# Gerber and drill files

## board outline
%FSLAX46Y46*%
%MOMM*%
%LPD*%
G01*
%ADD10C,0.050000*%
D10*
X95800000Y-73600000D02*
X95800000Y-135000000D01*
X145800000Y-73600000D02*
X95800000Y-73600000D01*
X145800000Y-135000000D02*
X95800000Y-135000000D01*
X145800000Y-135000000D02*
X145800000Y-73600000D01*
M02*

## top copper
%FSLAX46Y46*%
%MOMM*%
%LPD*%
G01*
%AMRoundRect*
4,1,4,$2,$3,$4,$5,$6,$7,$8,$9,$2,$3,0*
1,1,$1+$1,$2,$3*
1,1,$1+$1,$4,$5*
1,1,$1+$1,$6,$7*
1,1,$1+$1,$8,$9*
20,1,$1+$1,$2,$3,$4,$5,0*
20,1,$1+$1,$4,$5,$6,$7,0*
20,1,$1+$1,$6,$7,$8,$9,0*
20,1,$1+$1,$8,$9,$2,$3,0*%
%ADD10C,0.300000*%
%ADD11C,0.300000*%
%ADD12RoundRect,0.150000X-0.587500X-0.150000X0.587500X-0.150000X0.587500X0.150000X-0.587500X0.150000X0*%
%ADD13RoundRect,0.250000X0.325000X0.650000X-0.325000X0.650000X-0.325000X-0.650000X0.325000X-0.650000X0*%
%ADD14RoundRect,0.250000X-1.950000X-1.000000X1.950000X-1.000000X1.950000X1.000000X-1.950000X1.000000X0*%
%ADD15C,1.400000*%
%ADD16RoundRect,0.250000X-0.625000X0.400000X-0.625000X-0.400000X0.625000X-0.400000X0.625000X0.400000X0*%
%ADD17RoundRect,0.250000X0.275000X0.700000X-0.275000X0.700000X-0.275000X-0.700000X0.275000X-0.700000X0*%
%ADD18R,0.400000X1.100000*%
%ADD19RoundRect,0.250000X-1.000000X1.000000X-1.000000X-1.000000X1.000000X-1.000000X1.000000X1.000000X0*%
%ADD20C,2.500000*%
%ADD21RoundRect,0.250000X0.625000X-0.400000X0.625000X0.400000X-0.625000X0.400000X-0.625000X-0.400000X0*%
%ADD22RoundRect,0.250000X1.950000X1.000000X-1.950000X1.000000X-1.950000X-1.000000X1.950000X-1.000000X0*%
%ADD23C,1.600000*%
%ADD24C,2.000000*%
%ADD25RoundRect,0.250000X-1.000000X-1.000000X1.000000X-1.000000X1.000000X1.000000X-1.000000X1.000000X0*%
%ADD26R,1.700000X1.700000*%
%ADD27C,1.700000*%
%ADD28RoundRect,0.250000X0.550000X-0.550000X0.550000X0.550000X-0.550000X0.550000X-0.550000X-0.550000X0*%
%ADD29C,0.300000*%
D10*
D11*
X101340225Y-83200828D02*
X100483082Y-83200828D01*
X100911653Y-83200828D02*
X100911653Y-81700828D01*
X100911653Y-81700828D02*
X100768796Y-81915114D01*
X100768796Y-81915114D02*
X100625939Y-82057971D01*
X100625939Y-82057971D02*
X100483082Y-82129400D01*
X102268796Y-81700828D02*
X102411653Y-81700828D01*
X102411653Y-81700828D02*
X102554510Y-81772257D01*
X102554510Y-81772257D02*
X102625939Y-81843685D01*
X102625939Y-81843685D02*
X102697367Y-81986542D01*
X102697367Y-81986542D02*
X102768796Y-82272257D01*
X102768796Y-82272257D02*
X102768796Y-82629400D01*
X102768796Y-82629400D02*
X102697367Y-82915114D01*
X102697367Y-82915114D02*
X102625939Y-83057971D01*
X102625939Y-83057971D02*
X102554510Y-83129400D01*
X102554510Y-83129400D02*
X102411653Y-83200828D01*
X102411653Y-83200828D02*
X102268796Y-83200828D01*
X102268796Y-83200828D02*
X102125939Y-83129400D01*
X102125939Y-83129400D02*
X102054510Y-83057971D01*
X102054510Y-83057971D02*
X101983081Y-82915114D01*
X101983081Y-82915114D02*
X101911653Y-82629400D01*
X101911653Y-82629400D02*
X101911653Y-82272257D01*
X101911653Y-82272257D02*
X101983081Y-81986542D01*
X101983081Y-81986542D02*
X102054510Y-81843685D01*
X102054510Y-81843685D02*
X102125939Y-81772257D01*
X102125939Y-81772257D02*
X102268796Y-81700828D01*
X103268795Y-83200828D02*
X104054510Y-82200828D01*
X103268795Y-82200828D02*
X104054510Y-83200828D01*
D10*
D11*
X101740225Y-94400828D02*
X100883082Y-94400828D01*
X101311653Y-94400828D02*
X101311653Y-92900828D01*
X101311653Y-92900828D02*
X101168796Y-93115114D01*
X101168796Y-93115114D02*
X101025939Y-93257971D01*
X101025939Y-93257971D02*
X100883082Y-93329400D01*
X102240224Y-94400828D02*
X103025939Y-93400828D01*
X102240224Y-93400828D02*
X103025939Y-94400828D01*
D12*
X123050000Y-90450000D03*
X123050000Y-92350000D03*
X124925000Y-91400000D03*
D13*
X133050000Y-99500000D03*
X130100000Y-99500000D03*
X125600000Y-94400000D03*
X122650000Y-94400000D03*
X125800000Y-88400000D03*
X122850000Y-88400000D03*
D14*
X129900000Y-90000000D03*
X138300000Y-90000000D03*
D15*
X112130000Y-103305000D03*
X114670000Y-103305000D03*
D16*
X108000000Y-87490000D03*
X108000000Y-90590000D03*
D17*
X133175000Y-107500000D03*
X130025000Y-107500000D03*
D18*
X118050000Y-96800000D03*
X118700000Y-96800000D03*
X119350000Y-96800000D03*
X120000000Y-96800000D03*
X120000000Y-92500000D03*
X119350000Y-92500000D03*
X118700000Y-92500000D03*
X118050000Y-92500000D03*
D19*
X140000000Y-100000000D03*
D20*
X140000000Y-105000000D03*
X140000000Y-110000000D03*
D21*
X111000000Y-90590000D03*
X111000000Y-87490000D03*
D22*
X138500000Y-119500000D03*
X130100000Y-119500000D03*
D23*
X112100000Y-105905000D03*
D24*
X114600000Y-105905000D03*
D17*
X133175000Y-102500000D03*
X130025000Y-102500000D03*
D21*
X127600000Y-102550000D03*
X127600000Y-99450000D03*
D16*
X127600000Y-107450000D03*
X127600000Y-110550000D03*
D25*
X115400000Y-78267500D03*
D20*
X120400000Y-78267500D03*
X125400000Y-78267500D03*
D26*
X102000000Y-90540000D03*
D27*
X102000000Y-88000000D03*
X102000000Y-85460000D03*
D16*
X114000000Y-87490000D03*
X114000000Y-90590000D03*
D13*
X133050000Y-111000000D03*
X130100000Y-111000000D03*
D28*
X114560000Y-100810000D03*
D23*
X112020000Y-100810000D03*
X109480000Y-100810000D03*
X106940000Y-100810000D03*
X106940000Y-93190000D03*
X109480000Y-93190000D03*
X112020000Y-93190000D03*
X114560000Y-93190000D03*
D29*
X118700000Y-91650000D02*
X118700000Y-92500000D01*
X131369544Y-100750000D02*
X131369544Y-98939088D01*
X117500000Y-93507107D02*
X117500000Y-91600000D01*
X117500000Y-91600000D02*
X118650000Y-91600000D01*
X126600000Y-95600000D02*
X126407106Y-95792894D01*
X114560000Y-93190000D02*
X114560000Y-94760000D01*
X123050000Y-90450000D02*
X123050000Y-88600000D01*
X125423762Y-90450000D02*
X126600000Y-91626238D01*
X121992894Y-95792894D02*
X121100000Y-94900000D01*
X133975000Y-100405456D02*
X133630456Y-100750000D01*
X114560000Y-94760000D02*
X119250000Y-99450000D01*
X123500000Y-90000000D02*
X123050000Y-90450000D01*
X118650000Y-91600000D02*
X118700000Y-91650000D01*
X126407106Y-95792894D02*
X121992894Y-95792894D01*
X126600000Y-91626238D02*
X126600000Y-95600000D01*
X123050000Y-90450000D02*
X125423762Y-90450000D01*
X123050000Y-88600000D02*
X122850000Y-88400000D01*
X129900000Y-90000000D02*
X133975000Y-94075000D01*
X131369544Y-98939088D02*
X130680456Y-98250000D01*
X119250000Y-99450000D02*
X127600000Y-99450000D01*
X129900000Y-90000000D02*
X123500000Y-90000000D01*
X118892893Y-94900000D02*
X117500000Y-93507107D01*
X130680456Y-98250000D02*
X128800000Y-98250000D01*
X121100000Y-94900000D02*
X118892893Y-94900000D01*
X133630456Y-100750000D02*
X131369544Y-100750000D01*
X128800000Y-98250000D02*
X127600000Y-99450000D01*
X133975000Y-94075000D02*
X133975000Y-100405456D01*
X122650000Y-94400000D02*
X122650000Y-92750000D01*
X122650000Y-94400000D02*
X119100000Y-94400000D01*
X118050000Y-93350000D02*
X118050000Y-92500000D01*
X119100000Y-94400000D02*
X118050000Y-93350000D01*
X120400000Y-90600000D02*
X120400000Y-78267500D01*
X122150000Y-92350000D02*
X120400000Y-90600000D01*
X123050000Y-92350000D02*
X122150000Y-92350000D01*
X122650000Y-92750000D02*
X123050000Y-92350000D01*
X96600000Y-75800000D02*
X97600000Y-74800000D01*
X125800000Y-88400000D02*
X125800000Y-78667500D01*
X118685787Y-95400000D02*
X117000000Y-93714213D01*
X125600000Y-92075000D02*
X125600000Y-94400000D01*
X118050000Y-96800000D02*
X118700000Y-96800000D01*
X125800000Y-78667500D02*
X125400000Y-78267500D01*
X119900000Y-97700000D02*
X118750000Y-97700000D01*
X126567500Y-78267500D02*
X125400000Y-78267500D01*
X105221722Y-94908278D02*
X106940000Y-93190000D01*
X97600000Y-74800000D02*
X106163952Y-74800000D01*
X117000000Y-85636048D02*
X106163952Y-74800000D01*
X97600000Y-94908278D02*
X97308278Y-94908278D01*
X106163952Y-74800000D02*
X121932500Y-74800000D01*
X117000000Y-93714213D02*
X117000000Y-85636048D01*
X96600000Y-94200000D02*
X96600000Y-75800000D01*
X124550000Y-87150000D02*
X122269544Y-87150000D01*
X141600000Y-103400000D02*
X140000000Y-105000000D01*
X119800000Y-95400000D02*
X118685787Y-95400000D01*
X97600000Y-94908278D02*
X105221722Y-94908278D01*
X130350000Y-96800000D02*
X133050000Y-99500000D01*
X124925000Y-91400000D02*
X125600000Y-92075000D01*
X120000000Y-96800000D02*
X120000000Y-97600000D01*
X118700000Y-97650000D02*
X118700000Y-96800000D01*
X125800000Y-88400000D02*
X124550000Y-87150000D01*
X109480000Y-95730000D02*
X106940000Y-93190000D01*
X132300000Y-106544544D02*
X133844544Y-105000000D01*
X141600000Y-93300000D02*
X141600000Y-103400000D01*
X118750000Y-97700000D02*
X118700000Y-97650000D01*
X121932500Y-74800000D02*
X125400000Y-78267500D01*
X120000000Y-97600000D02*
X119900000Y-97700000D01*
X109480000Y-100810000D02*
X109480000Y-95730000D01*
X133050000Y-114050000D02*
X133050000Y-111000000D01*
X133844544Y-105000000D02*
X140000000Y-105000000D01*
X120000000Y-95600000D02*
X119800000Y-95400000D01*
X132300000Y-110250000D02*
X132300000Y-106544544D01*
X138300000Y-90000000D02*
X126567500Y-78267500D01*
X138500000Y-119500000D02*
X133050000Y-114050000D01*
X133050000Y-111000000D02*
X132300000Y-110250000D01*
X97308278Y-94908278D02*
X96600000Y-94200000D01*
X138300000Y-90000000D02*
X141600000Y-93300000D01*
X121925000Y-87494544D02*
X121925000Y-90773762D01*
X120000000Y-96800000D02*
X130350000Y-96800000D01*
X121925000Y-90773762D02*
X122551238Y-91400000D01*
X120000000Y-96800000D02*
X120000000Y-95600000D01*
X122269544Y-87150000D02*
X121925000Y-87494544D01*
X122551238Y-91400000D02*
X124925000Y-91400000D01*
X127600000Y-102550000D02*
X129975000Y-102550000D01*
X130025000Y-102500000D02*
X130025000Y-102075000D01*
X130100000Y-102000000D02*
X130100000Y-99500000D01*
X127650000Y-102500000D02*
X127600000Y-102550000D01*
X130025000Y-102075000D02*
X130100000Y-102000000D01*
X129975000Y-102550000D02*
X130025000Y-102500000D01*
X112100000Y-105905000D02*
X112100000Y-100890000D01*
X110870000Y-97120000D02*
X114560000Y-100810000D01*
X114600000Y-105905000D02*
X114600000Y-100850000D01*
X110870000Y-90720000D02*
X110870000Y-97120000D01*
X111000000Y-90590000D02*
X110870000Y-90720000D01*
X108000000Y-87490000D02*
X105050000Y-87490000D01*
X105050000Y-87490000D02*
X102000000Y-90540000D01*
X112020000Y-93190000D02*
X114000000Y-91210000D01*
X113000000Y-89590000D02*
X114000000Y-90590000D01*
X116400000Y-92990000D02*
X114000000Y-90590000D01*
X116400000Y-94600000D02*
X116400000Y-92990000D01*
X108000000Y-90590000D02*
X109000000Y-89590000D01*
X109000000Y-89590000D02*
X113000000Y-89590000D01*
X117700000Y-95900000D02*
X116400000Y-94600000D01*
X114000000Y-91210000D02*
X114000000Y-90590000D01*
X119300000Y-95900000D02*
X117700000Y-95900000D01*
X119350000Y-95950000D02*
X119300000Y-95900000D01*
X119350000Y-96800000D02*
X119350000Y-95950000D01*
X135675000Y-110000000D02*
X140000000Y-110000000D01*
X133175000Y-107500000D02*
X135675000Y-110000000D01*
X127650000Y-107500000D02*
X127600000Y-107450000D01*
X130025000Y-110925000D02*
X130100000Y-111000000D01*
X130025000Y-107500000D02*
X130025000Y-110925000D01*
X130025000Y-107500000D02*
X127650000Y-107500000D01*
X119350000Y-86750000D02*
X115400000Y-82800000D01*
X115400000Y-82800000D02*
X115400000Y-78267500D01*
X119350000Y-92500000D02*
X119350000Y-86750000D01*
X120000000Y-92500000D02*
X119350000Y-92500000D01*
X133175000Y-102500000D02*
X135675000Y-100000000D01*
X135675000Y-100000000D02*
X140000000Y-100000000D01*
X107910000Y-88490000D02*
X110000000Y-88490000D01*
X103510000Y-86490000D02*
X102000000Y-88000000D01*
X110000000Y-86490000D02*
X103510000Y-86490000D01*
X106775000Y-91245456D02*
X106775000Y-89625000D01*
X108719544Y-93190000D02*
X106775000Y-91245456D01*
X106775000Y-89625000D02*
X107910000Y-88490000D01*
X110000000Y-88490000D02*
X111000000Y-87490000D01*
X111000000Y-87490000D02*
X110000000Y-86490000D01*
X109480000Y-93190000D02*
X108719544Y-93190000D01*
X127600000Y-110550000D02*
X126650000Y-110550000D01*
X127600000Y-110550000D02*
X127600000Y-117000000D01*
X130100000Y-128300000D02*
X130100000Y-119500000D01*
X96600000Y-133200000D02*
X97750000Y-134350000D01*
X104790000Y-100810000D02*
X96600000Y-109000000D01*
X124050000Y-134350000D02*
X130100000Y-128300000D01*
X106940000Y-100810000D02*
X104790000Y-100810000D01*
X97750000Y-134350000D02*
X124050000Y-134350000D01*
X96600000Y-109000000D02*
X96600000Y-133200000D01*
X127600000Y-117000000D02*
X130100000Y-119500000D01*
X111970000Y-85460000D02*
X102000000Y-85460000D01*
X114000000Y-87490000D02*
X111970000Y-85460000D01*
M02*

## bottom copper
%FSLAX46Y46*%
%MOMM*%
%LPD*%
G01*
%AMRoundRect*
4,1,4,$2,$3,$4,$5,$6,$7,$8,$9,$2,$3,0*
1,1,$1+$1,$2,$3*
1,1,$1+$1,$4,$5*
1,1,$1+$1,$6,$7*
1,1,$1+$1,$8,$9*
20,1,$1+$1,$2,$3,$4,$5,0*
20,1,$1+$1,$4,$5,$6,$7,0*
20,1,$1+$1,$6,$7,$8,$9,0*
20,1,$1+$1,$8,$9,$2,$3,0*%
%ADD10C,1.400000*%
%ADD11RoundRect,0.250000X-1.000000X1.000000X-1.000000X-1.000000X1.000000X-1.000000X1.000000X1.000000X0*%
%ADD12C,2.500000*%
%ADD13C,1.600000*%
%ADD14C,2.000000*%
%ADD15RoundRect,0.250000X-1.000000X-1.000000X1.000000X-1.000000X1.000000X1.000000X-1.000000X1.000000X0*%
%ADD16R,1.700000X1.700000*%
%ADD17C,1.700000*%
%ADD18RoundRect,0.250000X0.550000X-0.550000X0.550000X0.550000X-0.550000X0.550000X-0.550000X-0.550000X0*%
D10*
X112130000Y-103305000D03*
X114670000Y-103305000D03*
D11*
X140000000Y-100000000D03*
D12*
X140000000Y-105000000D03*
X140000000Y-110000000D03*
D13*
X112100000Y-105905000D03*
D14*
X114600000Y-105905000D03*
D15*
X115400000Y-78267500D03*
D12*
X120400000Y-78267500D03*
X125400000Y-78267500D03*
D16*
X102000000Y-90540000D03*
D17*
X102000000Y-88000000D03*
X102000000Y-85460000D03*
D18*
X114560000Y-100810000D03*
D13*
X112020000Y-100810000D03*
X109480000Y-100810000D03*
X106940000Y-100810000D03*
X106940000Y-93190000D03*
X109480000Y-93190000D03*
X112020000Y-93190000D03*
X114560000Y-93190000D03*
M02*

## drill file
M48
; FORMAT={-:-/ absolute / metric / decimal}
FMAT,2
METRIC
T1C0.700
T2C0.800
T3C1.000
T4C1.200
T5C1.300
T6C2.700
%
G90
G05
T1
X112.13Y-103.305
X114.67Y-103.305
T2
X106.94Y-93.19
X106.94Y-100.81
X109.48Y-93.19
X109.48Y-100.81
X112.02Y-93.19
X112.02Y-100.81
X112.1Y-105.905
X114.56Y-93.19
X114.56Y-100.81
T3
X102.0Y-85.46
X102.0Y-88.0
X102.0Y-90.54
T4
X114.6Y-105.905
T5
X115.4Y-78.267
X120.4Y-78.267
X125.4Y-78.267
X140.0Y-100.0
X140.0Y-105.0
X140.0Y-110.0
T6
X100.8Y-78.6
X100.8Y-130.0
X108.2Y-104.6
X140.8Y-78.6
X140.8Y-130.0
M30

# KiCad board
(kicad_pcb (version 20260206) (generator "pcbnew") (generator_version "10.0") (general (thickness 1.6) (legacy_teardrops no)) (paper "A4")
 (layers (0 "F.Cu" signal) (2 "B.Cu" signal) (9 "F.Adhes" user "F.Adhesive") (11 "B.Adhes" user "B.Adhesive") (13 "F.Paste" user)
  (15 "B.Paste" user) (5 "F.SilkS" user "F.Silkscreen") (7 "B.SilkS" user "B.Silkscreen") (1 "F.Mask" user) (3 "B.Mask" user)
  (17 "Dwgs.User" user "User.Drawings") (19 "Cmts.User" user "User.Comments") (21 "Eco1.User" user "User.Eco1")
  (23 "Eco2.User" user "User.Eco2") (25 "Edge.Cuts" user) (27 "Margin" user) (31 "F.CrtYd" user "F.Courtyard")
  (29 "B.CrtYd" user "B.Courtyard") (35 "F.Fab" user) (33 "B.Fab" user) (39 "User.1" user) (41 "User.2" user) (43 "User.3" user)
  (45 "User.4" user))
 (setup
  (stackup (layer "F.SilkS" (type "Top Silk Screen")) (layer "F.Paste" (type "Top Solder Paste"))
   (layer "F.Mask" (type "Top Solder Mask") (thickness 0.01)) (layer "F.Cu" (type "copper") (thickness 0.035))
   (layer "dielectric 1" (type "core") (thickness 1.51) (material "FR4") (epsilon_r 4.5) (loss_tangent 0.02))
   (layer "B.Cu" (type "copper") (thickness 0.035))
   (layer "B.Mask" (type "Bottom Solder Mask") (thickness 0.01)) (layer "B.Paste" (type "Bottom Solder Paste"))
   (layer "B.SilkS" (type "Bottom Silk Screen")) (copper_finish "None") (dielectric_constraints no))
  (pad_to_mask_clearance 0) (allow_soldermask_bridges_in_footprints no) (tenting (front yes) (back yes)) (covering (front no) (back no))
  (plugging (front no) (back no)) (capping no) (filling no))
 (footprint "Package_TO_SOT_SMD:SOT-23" (layer "F.Cu") (at 123.9875 91.4)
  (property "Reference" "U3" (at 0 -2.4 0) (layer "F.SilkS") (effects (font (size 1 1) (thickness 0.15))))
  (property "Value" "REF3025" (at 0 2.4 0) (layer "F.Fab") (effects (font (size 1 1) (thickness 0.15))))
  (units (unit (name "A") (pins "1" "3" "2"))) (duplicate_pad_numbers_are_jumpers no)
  (pad "1" smd roundrect (at -0.9375 -0.95) (size 1.475 0.6) (layers "F.Cu" "F.Mask" "F.Paste") (roundrect_rratio 0.25) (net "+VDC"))
  (pad "2" smd roundrect (at -0.9375 0.95) (size 1.475 0.6) (layers "F.Cu" "F.Mask" "F.Paste") (roundrect_rratio 0.25) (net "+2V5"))
  (pad "3" smd roundrect (at 0.9375 0) (size 1.475 0.6) (layers "F.Cu" "F.Mask" "F.Paste") (roundrect_rratio 0.25) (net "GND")))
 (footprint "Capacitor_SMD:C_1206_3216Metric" (layer "F.Cu") (at 131.575 99.5 180)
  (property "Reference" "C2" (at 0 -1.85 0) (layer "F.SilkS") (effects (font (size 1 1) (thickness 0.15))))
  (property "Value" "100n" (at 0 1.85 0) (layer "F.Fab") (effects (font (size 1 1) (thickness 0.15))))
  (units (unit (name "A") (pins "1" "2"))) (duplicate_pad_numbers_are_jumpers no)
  (pad "1" smd roundrect (at -1.475 0 180) (size 1.15 1.8) (layers "F.Cu" "F.Mask" "F.Paste") (roundrect_rratio 0.217391) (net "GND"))
  (pad "2" smd roundrect (at 1.475 0 180) (size 1.15 1.8) (layers "F.Cu" "F.Mask" "F.Paste") (roundrect_rratio 0.217391)
   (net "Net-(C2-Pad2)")))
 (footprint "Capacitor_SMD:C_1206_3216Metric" (layer "F.Cu") (at 124.125 94.4 180)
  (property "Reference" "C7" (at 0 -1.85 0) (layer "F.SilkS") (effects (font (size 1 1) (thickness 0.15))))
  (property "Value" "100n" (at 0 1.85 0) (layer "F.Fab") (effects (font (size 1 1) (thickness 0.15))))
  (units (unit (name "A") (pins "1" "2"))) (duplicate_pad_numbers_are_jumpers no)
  (pad "1" smd roundrect (at -1.475 0 180) (size 1.15 1.8) (layers "F.Cu" "F.Mask" "F.Paste") (roundrect_rratio 0.217391) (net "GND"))
  (pad "2" smd roundrect (at 1.475 0 180) (size 1.15 1.8) (layers "F.Cu" "F.Mask" "F.Paste") (roundrect_rratio 0.217391) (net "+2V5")))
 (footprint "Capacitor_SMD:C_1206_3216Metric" (layer "F.Cu") (at 124.325 88.4 180)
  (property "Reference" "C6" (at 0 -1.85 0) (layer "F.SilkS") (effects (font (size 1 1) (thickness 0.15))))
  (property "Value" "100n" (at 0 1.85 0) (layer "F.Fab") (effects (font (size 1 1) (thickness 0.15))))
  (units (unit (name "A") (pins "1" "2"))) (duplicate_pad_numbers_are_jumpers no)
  (pad "1" smd roundrect (at -1.475 0 180) (size 1.15 1.8) (layers "F.Cu" "F.Mask" "F.Paste") (roundrect_rratio 0.217391) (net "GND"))
  (pad "2" smd roundrect (at 1.475 0 180) (size 1.15 1.8) (layers "F.Cu" "F.Mask" "F.Paste") (roundrect_rratio 0.217391) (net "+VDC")))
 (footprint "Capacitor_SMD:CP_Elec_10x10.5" (layer "F.Cu") (at 134.1 90)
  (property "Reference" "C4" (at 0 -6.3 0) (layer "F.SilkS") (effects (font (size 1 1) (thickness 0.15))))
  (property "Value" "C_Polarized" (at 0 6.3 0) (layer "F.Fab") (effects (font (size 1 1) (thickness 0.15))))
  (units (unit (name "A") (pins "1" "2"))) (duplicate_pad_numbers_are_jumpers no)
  (pad "1" smd roundrect (at -4.2 0) (size 4.4 2.5) (layers "F.Cu" "F.Mask" "F.Paste") (roundrect_rratio 0.1) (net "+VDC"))
  (pad "2" smd roundrect (at 4.2 0) (size 4.4 2.5) (layers "F.Cu" "F.Mask" "F.Paste") (roundrect_rratio 0.1) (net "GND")))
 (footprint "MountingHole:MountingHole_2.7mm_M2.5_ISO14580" (layer "F.Cu") (at 140.8 130 90)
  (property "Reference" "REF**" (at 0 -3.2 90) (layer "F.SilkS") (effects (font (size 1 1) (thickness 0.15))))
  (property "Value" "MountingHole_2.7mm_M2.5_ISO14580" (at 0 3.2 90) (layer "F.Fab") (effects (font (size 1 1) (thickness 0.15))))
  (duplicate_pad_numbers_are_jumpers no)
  (pad "" np_thru_hole circle (at 0 0 90) (size 2.7 2.7) (drill 2.7) (layers "*.Cu" "*.Mask")))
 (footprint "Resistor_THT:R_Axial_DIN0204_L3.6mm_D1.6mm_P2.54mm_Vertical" (layer "F.Cu") (at 112.13 103.305)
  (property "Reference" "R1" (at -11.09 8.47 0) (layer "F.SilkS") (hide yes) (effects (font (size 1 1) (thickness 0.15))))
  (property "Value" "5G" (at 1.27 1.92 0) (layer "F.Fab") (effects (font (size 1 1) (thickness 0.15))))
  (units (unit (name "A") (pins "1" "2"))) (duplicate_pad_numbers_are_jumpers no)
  (pad "1" thru_hole circle (at 0 0) (size 1.4 1.4) (drill 0.7) (layers "*.Cu" "*.Mask") (remove_unused_layers no) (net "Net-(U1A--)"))
  (pad "2" thru_hole circle (at 2.54 0) (size 1.4 1.4) (drill 0.7) (layers "*.Cu" "*.Mask") (remove_unused_layers no) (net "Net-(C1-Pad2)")))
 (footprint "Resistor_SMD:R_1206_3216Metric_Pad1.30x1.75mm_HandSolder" (layer "F.Cu") (at 108 89.04 -90)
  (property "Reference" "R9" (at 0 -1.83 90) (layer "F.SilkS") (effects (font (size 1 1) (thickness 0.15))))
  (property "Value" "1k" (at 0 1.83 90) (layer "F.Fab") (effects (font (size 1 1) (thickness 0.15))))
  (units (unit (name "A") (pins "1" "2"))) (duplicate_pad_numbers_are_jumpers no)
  (pad "1" smd roundrect (at -1.55 0 270) (size 1.3 1.75) (layers "F.Cu" "F.Mask" "F.Paste") (roundrect_rratio 0.192308)
   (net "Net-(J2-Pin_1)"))
  (pad "2" smd roundrect (at 1.55 0 270) (size 1.3 1.75) (layers "F.Cu" "F.Mask" "F.Paste") (roundrect_rratio 0.192308)
   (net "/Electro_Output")))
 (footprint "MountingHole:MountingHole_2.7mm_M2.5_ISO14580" (layer "F.Cu") (at 100.8 78.6 90)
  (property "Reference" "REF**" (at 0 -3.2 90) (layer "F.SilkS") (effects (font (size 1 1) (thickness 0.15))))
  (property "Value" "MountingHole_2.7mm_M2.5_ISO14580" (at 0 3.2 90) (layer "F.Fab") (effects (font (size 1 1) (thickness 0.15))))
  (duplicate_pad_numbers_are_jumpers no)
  (pad "" np_thru_hole circle (at 0 0 90) (size 2.7 2.7) (drill 2.7) (layers "*.Cu" "*.Mask")))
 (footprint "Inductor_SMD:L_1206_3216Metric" (layer "F.Cu") (at 131.6 107.5 180)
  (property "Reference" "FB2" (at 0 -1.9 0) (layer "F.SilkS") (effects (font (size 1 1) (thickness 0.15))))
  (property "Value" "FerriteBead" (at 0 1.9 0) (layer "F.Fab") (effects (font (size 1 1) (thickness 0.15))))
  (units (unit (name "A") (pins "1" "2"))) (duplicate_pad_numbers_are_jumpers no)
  (pad "1" smd roundrect (at -1.575 0 180) (size 1.05 1.9) (layers "F.Cu" "F.Mask" "F.Paste") (roundrect_rratio 0.238095) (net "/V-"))
  (pad "2" smd roundrect (at 1.575 0 180) (size 1.05 1.9) (layers "F.Cu" "F.Mask" "F.Paste") (roundrect_rratio 0.238095)
   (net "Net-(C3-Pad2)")))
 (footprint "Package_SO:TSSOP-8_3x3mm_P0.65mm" (layer "F.Cu") (at 119.025 94.65 90)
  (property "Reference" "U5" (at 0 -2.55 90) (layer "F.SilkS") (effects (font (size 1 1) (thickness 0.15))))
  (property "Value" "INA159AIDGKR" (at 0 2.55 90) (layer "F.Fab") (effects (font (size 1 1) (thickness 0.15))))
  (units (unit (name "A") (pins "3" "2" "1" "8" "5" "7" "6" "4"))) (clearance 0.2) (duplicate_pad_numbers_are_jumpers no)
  (pad "1" smd rect (at -2.15 -0.975 90) (size 1.1 0.4) (layers "F.Cu" "F.Mask" "F.Paste") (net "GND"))
  (pad "2" smd rect (at -2.15 -0.325 90) (size 1.1 0.4) (layers "F.Cu" "F.Mask" "F.Paste") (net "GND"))
  (pad "3" smd rect (at -2.15 0.325 90) (size 1.1 0.4) (layers "F.Cu" "F.Mask" "F.Paste") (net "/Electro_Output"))
  (pad "4" smd rect (at -2.15 0.975 90) (size 1.1 0.4) (layers "F.Cu" "F.Mask" "F.Paste") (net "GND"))
  (pad "5" smd rect (at 2.15 0.975 90) (size 1.1 0.4) (layers "F.Cu" "F.Mask" "F.Paste") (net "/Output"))
  (pad "6" smd rect (at 2.15 0.325 90) (size 1.1 0.4) (layers "F.Cu" "F.Mask" "F.Paste") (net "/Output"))
  (pad "7" smd rect (at 2.15 -0.325 90) (size 1.1 0.4) (layers "F.Cu" "F.Mask" "F.Paste") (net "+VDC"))
  (pad "8" smd rect (at 2.15 -0.975 90) (size 1.1 0.4) (layers "F.Cu" "F.Mask" "F.Paste") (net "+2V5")))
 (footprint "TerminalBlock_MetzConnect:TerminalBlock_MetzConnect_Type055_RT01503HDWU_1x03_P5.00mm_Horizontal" (layer "F.Cu")
  (at 140 100 -90)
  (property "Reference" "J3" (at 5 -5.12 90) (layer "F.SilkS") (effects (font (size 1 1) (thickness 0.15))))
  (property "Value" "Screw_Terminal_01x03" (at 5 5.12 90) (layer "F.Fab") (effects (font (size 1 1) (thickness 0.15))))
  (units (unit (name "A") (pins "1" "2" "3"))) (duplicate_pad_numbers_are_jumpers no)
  (pad "1" thru_hole roundrect (at 0 0 270) (size 2.5 2.5) (drill 1.3) (layers "*.Cu" "*.Mask") (remove_unused_layers no)
   (roundrect_rratio 0.1) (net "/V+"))
  (pad "2" thru_hole circle (at 5 0 270) (size 2.5 2.5) (drill 1.3) (layers "*.Cu" "*.Mask") (remove_unused_layers no) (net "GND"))
  (pad "3" thru_hole circle (at 10 0 270) (size 2.5 2.5) (drill 1.3) (layers "*.Cu" "*.Mask") (remove_unused_layers no) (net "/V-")))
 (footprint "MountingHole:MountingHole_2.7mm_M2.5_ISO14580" (layer "F.Cu") (at 100.8 130 90)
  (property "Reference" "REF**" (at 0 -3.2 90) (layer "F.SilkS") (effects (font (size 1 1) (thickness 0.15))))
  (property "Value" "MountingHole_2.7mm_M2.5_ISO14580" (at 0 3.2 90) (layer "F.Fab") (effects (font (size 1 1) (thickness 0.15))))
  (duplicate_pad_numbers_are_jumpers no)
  (pad "" np_thru_hole circle (at 0 0 90) (size 2.7 2.7) (drill 2.7) (layers "*.Cu" "*.Mask")))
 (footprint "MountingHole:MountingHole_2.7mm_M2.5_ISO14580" (layer "F.Cu") (at 108.2 104.6 180)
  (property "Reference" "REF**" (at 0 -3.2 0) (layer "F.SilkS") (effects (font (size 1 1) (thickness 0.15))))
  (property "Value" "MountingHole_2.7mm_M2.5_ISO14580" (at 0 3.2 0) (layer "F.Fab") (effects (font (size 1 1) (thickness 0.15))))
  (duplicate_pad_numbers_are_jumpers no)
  (pad "" np_thru_hole circle (at 0 0 180) (size 2.7 2.7) (drill 2.7) (layers "*.Cu" "*.Mask")))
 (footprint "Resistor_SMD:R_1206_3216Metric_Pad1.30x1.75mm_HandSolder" (layer "F.Cu") (at 111 89.04 90)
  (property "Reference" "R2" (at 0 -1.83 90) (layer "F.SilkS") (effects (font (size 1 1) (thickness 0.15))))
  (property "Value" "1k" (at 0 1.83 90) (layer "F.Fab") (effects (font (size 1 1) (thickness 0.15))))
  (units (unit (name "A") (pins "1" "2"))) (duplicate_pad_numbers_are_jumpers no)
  (pad "1" smd roundrect (at -1.55 0 90) (size 1.3 1.75) (layers "F.Cu" "F.Mask" "F.Paste") (roundrect_rratio 0.192308)
   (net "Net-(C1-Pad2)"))
  (pad "2" smd roundrect (at 1.55 0 90) (size 1.3 1.75) (layers "F.Cu" "F.Mask" "F.Paste") (roundrect_rratio 0.192308)
   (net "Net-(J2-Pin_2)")))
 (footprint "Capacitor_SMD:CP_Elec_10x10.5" (layer "F.Cu") (at 134.3 119.5 180)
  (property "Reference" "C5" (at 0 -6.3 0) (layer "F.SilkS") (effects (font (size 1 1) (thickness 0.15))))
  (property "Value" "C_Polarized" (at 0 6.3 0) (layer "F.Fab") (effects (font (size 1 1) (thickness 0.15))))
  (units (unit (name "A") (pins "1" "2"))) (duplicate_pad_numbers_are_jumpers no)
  (pad "1" smd roundrect (at -4.2 0 180) (size 4.4 2.5) (layers "F.Cu" "F.Mask" "F.Paste") (roundrect_rratio 0.1) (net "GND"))
  (pad "2" smd roundrect (at 4.2 0 180) (size 4.4 2.5) (layers "F.Cu" "F.Mask" "F.Paste") (roundrect_rratio 0.1) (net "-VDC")))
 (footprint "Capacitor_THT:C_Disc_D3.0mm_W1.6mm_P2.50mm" (layer "F.Cu") (at 112.1 105.905)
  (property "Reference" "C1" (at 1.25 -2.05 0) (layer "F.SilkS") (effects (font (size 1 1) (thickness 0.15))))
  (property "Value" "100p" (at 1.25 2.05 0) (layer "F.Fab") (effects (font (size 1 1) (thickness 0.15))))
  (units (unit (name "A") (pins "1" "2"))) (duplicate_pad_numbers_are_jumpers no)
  (pad "1" thru_hole circle (at 0 0) (size 1.6 1.6) (drill 0.8) (layers "*.Cu" "*.Mask") (remove_unused_layers no) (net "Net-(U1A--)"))
  (pad "2" thru_hole circle (at 2.5 0) (size 2 2) (drill 1.2) (layers "*.Cu" "*.Mask") (remove_unused_layers no) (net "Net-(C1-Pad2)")))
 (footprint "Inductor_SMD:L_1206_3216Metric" (layer "F.Cu") (at 131.6 102.5 180)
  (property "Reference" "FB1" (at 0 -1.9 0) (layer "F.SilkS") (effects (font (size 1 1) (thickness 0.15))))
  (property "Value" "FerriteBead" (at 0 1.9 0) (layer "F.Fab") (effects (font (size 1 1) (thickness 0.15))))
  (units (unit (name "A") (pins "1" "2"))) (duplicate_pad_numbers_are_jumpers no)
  (pad "1" smd roundrect (at -1.575 0 180) (size 1.05 1.9) (layers "F.Cu" "F.Mask" "F.Paste") (roundrect_rratio 0.238095) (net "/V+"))
  (pad "2" smd roundrect (at 1.575 0 180) (size 1.05 1.9) (layers "F.Cu" "F.Mask" "F.Paste") (roundrect_rratio 0.238095)
   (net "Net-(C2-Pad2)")))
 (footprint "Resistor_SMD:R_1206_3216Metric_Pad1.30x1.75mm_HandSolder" (layer "F.Cu") (at 127.6 101 90)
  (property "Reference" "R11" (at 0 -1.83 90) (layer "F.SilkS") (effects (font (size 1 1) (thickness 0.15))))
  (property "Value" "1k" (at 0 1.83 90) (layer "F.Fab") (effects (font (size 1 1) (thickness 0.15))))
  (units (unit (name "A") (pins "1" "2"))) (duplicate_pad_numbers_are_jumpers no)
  (pad "1" smd roundrect (at -1.55 0 90) (size 1.3 1.75) (layers "F.Cu" "F.Mask" "F.Paste") (roundrect_rratio 0.192308)
   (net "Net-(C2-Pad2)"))
  (pad "2" smd roundrect (at 1.55 0 90) (size 1.3 1.75) (layers "F.Cu" "F.Mask" "F.Paste") (roundrect_rratio 0.192308) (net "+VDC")))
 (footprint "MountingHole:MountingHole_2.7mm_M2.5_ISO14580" (layer "F.Cu") (at 140.8 78.6 90)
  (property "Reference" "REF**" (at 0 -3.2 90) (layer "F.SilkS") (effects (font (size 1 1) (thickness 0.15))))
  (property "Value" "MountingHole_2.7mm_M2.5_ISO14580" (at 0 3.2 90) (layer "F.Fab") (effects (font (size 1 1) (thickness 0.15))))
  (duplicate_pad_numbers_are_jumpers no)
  (pad "" np_thru_hole circle (at 0 0 90) (size 2.7 2.7) (drill 2.7) (layers "*.Cu" "*.Mask")))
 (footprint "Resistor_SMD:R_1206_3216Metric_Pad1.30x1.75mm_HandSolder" (layer "F.Cu") (at 127.6 109 -90)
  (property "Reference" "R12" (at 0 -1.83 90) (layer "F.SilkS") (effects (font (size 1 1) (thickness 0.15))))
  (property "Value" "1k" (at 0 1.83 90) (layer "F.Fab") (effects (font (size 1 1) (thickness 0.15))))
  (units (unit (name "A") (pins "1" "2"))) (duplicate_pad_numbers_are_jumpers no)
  (pad "1" smd roundrect (at -1.55 0 270) (size 1.3 1.75) (layers "F.Cu" "F.Mask" "F.Paste") (roundrect_rratio 0.192308)
   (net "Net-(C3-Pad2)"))
  (pad "2" smd roundrect (at 1.55 0 270) (size 1.3 1.75) (layers "F.Cu" "F.Mask" "F.Paste") (roundrect_rratio 0.192308) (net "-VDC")))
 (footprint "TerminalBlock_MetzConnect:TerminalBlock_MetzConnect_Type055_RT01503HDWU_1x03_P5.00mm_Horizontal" (layer "F.Cu")
  (at 115.4 78.2675)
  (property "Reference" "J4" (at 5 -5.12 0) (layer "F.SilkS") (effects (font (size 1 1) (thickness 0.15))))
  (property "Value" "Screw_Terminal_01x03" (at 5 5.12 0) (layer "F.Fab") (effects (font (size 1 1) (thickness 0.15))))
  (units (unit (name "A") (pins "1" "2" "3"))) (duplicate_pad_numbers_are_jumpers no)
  (pad "1" thru_hole roundrect (at 0 0) (size 2.5 2.5) (drill 1.3) (layers "*.Cu" "*.Mask") (remove_unused_layers no) (roundrect_rratio 0.1)
   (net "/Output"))
  (pad "2" thru_hole circle (at 5 0) (size 2.5 2.5) (drill 1.3) (layers "*.Cu" "*.Mask") (remove_unused_layers no) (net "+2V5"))
  (pad "3" thru_hole circle (at 10 0) (size 2.5 2.5) (drill 1.3) (layers "*.Cu" "*.Mask") (remove_unused_layers no) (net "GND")))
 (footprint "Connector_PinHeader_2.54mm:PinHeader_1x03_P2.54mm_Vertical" (layer "F.Cu") (at 102 90.54 180)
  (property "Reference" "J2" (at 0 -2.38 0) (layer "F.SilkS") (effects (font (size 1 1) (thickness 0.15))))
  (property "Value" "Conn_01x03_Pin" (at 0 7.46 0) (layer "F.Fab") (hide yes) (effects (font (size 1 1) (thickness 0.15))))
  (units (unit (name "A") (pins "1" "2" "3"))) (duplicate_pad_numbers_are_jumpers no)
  (pad "1" thru_hole rect (at 0 0 180) (size 1.7 1.7) (drill 1) (layers "*.Cu" "*.Mask") (remove_unused_layers no) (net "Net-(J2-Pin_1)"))
  (pad "2" thru_hole circle (at 0 2.54 180) (size 1.7 1.7) (drill 1) (layers "*.Cu" "*.Mask") (remove_unused_layers no)
   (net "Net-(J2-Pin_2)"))
  (pad "3" thru_hole circle (at 0 5.08 180) (size 1.7 1.7) (drill 1) (layers "*.Cu" "*.Mask") (remove_unused_layers no)
   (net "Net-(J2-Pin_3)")))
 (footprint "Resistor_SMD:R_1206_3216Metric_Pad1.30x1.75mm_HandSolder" (layer "F.Cu") (at 114 89.04 -90)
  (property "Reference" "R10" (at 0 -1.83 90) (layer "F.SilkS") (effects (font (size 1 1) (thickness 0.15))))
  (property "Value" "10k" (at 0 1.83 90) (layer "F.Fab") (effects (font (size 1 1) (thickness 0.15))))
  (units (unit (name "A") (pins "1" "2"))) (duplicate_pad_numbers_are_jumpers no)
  (pad "1" smd roundrect (at -1.55 0 270) (size 1.3 1.75) (layers "F.Cu" "F.Mask" "F.Paste") (roundrect_rratio 0.192308)
   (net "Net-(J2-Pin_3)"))
  (pad "2" smd roundrect (at 1.55 0 270) (size 1.3 1.75) (layers "F.Cu" "F.Mask" "F.Paste") (roundrect_rratio 0.192308)
   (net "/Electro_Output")))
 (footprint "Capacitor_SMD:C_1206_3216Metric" (layer "F.Cu") (at 131.575 111 180)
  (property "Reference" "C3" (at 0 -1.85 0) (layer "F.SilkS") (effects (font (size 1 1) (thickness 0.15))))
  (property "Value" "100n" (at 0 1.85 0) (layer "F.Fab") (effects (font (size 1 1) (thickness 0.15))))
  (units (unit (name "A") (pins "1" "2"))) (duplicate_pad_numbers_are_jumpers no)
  (pad "1" smd roundrect (at -1.475 0 180) (size 1.15 1.8) (layers "F.Cu" "F.Mask" "F.Paste") (roundrect_rratio 0.217391) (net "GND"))
  (pad "2" smd roundrect (at 1.475 0 180) (size 1.15 1.8) (layers "F.Cu" "F.Mask" "F.Paste") (roundrect_rratio 0.217391)
   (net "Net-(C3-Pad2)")))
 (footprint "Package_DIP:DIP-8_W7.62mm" (layer "B.Cu") (at 114.56 100.81 90)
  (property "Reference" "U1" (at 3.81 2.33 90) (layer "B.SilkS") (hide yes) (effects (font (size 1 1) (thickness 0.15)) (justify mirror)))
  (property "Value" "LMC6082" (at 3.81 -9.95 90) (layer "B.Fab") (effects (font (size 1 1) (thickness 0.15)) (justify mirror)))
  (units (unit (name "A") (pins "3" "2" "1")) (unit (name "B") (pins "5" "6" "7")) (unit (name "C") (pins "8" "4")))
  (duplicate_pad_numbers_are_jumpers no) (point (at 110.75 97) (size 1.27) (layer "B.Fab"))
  (pad "1" thru_hole roundrect (at 0 0 90) (size 1.6 1.6) (drill 0.8) (layers "*.Cu" "*.Mask") (remove_unused_layers no)
   (roundrect_rratio 0.15625) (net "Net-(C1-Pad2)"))
  (pad "2" thru_hole circle (at 0 -2.54 90) (size 1.6 1.6) (drill 0.8) (layers "*.Cu" "*.Mask") (remove_unused_layers no)
   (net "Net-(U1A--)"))
  (pad "3" thru_hole circle (at 0 -5.08 90) (size 1.6 1.6) (drill 0.8) (layers "*.Cu" "*.Mask") (remove_unused_layers no) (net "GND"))
  (pad "4" thru_hole circle (at 0 -7.62 90) (size 1.6 1.6) (drill 0.8) (layers "*.Cu" "*.Mask") (remove_unused_layers no) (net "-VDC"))
  (pad "5" thru_hole circle (at 7.62 -7.62 90) (size 1.6 1.6) (drill 0.8) (layers "*.Cu" "*.Mask") (remove_unused_layers no) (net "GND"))
  (pad "6" thru_hole circle (at 7.62 -5.08 90) (size 1.6 1.6) (drill 0.8) (layers "*.Cu" "*.Mask") (remove_unused_layers no)
   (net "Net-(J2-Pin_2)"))
  (pad "7" thru_hole circle (at 7.62 -2.54 90) (size 1.6 1.6) (drill 0.8) (layers "*.Cu" "*.Mask") (remove_unused_layers no)
   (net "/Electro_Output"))
  (pad "8" thru_hole circle (at 7.62 0 90) (size 1.6 1.6) (drill 0.8) (layers "*.Cu" "*.Mask") (remove_unused_layers no) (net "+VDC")))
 (gr_line (start 95.8 73.6) (end 95.8 135) (stroke (width 0.05) (type default)) (layer "Edge.Cuts"))
 (gr_line (start 145.8 73.6) (end 95.8 73.6) (stroke (width 0.05) (type default)) (layer "Edge.Cuts"))
 (gr_line (start 145.8 135) (end 95.8 135) (stroke (width 0.05) (type default)) (layer "Edge.Cuts"))
 (gr_line (start 145.8 135) (end 145.8 73.6) (stroke (width 0.05) (type default)) (layer "Edge.Cuts"))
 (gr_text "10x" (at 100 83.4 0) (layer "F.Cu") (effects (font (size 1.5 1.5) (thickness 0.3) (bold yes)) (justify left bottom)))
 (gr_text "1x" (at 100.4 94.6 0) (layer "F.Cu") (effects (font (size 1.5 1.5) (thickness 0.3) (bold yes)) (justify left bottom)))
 (segment (start 118.7 91.65) (end 118.7 92.5) (width 0.3) (layer "F.Cu") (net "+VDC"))
 (segment (start 131.369544 100.75) (end 131.369544 98.939088) (width 0.3) (layer "F.Cu") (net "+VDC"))
 (segment (start 117.5 93.507107) (end 117.5 91.6) (width 0.3) (layer "F.Cu") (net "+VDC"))
 (segment (start 117.5 91.6) (end 118.65 91.6) (width 0.3) (layer "F.Cu") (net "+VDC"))
 (segment (start 126.6 95.6) (end 126.407106 95.792894) (width 0.3) (layer "F.Cu") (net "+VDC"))
 (segment (start 114.56 93.19) (end 114.56 94.76) (width 0.3) (layer "F.Cu") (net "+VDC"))
 (segment (start 123.05 90.45) (end 123.05 88.6) (width 0.3) (layer "F.Cu") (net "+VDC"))
 (segment (start 125.423762 90.45) (end 126.6 91.626238) (width 0.3) (layer "F.Cu") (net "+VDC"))
 (segment (start 121.992894 95.792894) (end 121.1 94.9) (width 0.3) (layer "F.Cu") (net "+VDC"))
 (segment (start 133.975 100.405456) (end 133.630456 100.75) (width 0.3) (layer "F.Cu") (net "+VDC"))
 (segment (start 114.56 94.76) (end 119.25 99.45) (width 0.3) (layer "F.Cu") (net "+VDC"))
 (segment (start 123.5 90) (end 123.05 90.45) (width 0.3) (layer "F.Cu") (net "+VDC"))
 (segment (start 118.65 91.6) (end 118.7 91.65) (width 0.3) (layer "F.Cu") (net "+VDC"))
 (segment (start 126.407106 95.792894) (end 121.992894 95.792894) (width 0.3) (layer "F.Cu") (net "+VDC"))
 (segment (start 126.6 91.626238) (end 126.6 95.6) (width 0.3) (layer "F.Cu") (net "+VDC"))
 (segment (start 123.05 90.45) (end 125.423762 90.45) (width 0.3) (layer "F.Cu") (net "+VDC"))
 (segment (start 123.05 88.6) (end 122.85 88.4) (width 0.3) (layer "F.Cu") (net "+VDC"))
 (segment (start 129.9 90) (end 133.975 94.075) (width 0.3) (layer "F.Cu") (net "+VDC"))
 (segment (start 131.369544 98.939088) (end 130.680456 98.25) (width 0.3) (layer "F.Cu") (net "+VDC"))
 (segment (start 119.25 99.45) (end 127.6 99.45) (width 0.3) (layer "F.Cu") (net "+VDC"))
 (segment (start 129.9 90) (end 123.5 90) (width 0.3) (layer "F.Cu") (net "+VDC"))
 (segment (start 118.892893 94.9) (end 117.5 93.507107) (width 0.3) (layer "F.Cu") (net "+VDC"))
 (segment (start 130.680456 98.25) (end 128.8 98.25) (width 0.3) (layer "F.Cu") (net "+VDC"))
 (segment (start 121.1 94.9) (end 118.892893 94.9) (width 0.3) (layer "F.Cu") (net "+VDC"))
 (segment (start 133.630456 100.75) (end 131.369544 100.75) (width 0.3) (layer "F.Cu") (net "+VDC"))
 (segment (start 128.8 98.25) (end 127.6 99.45) (width 0.3) (layer "F.Cu") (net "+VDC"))
 (segment (start 133.975 94.075) (end 133.975 100.405456) (width 0.3) (layer "F.Cu") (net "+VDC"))
 (segment (start 122.65 94.4) (end 122.65 92.75) (width 0.3) (layer "F.Cu") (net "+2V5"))
 (segment (start 122.65 94.4) (end 119.1 94.4) (width 0.3) (layer "F.Cu") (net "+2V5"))
 (segment (start 118.05 93.35) (end 118.05 92.5) (width 0.3) (layer "F.Cu") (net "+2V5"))
 (segment (start 119.1 94.4) (end 118.05 93.35) (width 0.3) (layer "F.Cu") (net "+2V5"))
 (segment (start 120.4 90.6) (end 120.4 78.2675) (width 0.3) (layer "F.Cu") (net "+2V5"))
 (segment (start 122.15 92.35) (end 120.4 90.6) (width 0.3) (layer "F.Cu") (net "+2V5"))
 (segment (start 123.05 92.35) (end 122.15 92.35) (width 0.3) (layer "F.Cu") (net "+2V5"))
 (segment (start 122.65 92.75) (end 123.05 92.35) (width 0.3) (layer "F.Cu") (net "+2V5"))
 (segment (start 96.6 75.8) (end 97.6 74.8) (width 0.3) (layer "F.Cu") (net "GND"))
 (segment (start 125.8 88.4) (end 125.8 78.6675) (width 0.3) (layer "F.Cu") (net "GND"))
 (segment (start 118.685787 95.4) (end 117 93.714213) (width 0.3) (layer "F.Cu") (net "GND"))
 (segment (start 125.6 92.075) (end 125.6 94.4) (width 0.3) (layer "F.Cu") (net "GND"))
 (segment (start 118.05 96.8) (end 118.7 96.8) (width 0.3) (layer "F.Cu") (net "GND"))
 (segment (start 125.8 78.6675) (end 125.4 78.2675) (width 0.3) (layer "F.Cu") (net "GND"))
 (segment (start 119.9 97.7) (end 118.75 97.7) (width 0.3) (layer "F.Cu") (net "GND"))
 (segment (start 126.5675 78.2675) (end 125.4 78.2675) (width 0.3) (layer "F.Cu") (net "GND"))
 (segment (start 105.221722 94.908278) (end 106.94 93.19) (width 0.3) (layer "F.Cu") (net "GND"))
 (segment (start 97.6 74.8) (end 106.163952 74.8) (width 0.3) (layer "F.Cu") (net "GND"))
 (segment (start 117 85.636048) (end 106.163952 74.8) (width 0.3) (layer "F.Cu") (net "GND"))
 (segment (start 97.6 94.908278) (end 97.308278 94.908278) (width 0.3) (layer "F.Cu") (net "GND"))
 (segment (start 106.163952 74.8) (end 121.9325 74.8) (width 0.3) (layer "F.Cu") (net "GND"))
 (segment (start 117 93.714213) (end 117 85.636048) (width 0.3) (layer "F.Cu") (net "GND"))
 (segment (start 96.6 94.2) (end 96.6 75.8) (width 0.3) (layer "F.Cu") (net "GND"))
 (segment (start 124.55 87.15) (end 122.269544 87.15) (width 0.3) (layer "F.Cu") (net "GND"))
 (segment (start 141.6 103.4) (end 140 105) (width 0.3) (layer "F.Cu") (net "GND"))
 (segment (start 119.8 95.4) (end 118.685787 95.4) (width 0.3) (layer "F.Cu") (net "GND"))
 (segment (start 97.6 94.908278) (end 105.221722 94.908278) (width 0.3) (layer "F.Cu") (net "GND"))
 (segment (start 130.35 96.8) (end 133.05 99.5) (width 0.3) (layer "F.Cu") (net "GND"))
 (segment (start 124.925 91.4) (end 125.6 92.075) (width 0.3) (layer "F.Cu") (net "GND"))
 (segment (start 120 96.8) (end 120 97.6) (width 0.3) (layer "F.Cu") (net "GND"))
 (segment (start 118.7 97.65) (end 118.7 96.8) (width 0.3) (layer "F.Cu") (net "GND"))
 (segment (start 125.8 88.4) (end 124.55 87.15) (width 0.3) (layer "F.Cu") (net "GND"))
 (segment (start 109.48 95.73) (end 106.94 93.19) (width 0.3) (layer "F.Cu") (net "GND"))
 (segment (start 132.3 106.544544) (end 133.844544 105) (width 0.3) (layer "F.Cu") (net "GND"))
 (segment (start 141.6 93.3) (end 141.6 103.4) (width 0.3) (layer "F.Cu") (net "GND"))
 (segment (start 118.75 97.7) (end 118.7 97.65) (width 0.3) (layer "F.Cu") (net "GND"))
 (segment (start 121.9325 74.8) (end 125.4 78.2675) (width 0.3) (layer "F.Cu") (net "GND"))
 (segment (start 120 97.6) (end 119.9 97.7) (width 0.3) (layer "F.Cu") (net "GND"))
 (segment (start 109.48 100.81) (end 109.48 95.73) (width 0.3) (layer "F.Cu") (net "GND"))
 (segment (start 133.05 114.05) (end 133.05 111) (width 0.3) (layer "F.Cu") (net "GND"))
 (segment (start 133.844544 105) (end 140 105) (width 0.3) (layer "F.Cu") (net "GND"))
 (segment (start 120 95.6) (end 119.8 95.4) (width 0.3) (layer "F.Cu") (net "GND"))
 (segment (start 132.3 110.25) (end 132.3 106.544544) (width 0.3) (layer "F.Cu") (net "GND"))
 (segment (start 138.3 90) (end 126.5675 78.2675) (width 0.3) (layer "F.Cu") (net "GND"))
 (segment (start 138.5 119.5) (end 133.05 114.05) (width 0.3) (layer "F.Cu") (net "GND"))
 (segment (start 133.05 111) (end 132.3 110.25) (width 0.3) (layer "F.Cu") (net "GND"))
 (segment (start 97.308278 94.908278) (end 96.6 94.2) (width 0.3) (layer "F.Cu") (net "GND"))
 (segment (start 138.3 90) (end 141.6 93.3) (width 0.3) (layer "F.Cu") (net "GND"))
 (segment (start 121.925 87.494544) (end 121.925 90.773762) (width 0.3) (layer "F.Cu") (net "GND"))
 (segment (start 120 96.8) (end 130.35 96.8) (width 0.3) (layer "F.Cu") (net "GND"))
 (segment (start 121.925 90.773762) (end 122.551238 91.4) (width 0.3) (layer "F.Cu") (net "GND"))
 (segment (start 120 96.8) (end 120 95.6) (width 0.3) (layer "F.Cu") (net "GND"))
 (segment (start 122.269544 87.15) (end 121.925 87.494544) (width 0.3) (layer "F.Cu") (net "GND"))
 (segment (start 122.551238 91.4) (end 124.925 91.4) (width 0.3) (layer "F.Cu") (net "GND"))
 (segment (start 127.6 102.55) (end 129.975 102.55) (width 0.3) (layer "F.Cu") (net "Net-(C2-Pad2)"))
 (segment (start 130.025 102.5) (end 130.025 102.075) (width 0.3) (layer "F.Cu") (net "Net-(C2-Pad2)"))
 (segment (start 130.1 102) (end 130.1 99.5) (width 0.3) (layer "F.Cu") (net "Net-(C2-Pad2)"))
 (segment (start 127.65 102.5) (end 127.6 102.55) (width 0.3) (layer "F.Cu") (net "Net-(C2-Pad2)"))
 (segment (start 130.025 102.075) (end 130.1 102) (width 0.3) (layer "F.Cu") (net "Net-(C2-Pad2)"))
 (segment (start 129.975 102.55) (end 130.025 102.5) (width 0.3) (layer "F.Cu") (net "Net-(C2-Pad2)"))
 (segment (start 112.1 105.905) (end 112.1 100.89) (width 0.3) (layer "F.Cu") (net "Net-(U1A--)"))
 (segment (start 110.87 97.12) (end 114.56 100.81) (width 0.3) (layer "F.Cu") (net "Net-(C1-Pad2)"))
 (segment (start 114.6 105.905) (end 114.6 100.85) (width 0.3) (layer "F.Cu") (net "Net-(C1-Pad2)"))
 (segment (start 110.87 90.72) (end 110.87 97.12) (width 0.3) (layer "F.Cu") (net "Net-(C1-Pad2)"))
 (segment (start 111 90.59) (end 110.87 90.72) (width 0.3) (layer "F.Cu") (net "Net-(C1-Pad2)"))
 (segment (start 108 87.49) (end 105.05 87.49) (width 0.3) (layer "F.Cu") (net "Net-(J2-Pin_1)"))
 (segment (start 105.05 87.49) (end 102 90.54) (width 0.3) (layer "F.Cu") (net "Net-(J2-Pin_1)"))
 (segment (start 112.02 93.19) (end 114 91.21) (width 0.3) (layer "F.Cu") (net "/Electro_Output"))
 (segment (start 113 89.59) (end 114 90.59) (width 0.3) (layer "F.Cu") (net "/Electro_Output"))
 (segment (start 116.4 92.99) (end 114 90.59) (width 0.3) (layer "F.Cu") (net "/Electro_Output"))
 (segment (start 116.4 94.6) (end 116.4 92.99) (width 0.3) (layer "F.Cu") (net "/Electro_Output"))
 (segment (start 108 90.59) (end 109 89.59) (width 0.3) (layer "F.Cu") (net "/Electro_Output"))
 (segment (start 109 89.59) (end 113 89.59) (width 0.3) (layer "F.Cu") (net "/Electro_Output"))
 (segment (start 117.7 95.9) (end 116.4 94.6) (width 0.3) (layer "F.Cu") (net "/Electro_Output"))
 (segment (start 114 91.21) (end 114 90.59) (width 0.3) (layer "F.Cu") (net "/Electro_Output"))
 (segment (start 119.3 95.9) (end 117.7 95.9) (width 0.3) (layer "F.Cu") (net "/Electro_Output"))
 (segment (start 119.35 95.95) (end 119.3 95.9) (width 0.3) (layer "F.Cu") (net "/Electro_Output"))
 (segment (start 119.35 96.8) (end 119.35 95.95) (width 0.3) (layer "F.Cu") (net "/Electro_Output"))
 (segment (start 135.675 110) (end 140 110) (width 0.3) (layer "F.Cu") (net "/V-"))
 (segment (start 133.175 107.5) (end 135.675 110) (width 0.3) (layer "F.Cu") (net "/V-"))
 (segment (start 127.65 107.5) (end 127.6 107.45) (width 0.3) (layer "F.Cu") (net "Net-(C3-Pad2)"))
 (segment (start 130.025 110.925) (end 130.1 111) (width 0.3) (layer "F.Cu") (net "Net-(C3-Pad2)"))
 (segment (start 130.025 107.5) (end 130.025 110.925) (width 0.3) (layer "F.Cu") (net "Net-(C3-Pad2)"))
 (segment (start 130.025 107.5) (end 127.65 107.5) (width 0.3) (layer "F.Cu") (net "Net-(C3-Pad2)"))
 (segment (start 119.35 86.75) (end 115.4 82.8) (width 0.3) (layer "F.Cu") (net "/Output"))
 (segment (start 115.4 82.8) (end 115.4 78.2675) (width 0.3) (layer "F.Cu") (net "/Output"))
 (segment (start 119.35 92.5) (end 119.35 86.75) (width 0.3) (layer "F.Cu") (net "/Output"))
 (segment (start 120 92.5) (end 119.35 92.5) (width 0.3) (layer "F.Cu") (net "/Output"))
 (segment (start 133.175 102.5) (end 135.675 100) (width 0.3) (layer "F.Cu") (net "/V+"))
 (segment (start 135.675 100) (end 140 100) (width 0.3) (layer "F.Cu") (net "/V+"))
 (segment (start 107.91 88.49) (end 110 88.49) (width 0.3) (layer "F.Cu") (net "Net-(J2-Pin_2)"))
 (segment (start 103.51 86.49) (end 102 88) (width 0.3) (layer "F.Cu") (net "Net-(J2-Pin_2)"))
 (segment (start 110 86.49) (end 103.51 86.49) (width 0.3) (layer "F.Cu") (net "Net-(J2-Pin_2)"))
 (segment (start 106.775 91.245456) (end 106.775 89.625) (width 0.3) (layer "F.Cu") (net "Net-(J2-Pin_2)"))
 (segment (start 108.719544 93.19) (end 106.775 91.245456) (width 0.3) (layer "F.Cu") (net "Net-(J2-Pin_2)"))
 (segment (start 106.775 89.625) (end 107.91 88.49) (width 0.3) (layer "F.Cu") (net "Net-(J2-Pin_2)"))
 (segment (start 110 88.49) (end 111 87.49) (width 0.3) (layer "F.Cu") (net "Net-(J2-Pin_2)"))
 (segment (start 111 87.49) (end 110 86.49) (width 0.3) (layer "F.Cu") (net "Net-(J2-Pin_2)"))
 (segment (start 109.48 93.19) (end 108.719544 93.19) (width 0.3) (layer "F.Cu") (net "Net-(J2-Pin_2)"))
 (segment (start 127.6 110.55) (end 126.65 110.55) (width 0.3) (layer "F.Cu") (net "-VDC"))
 (segment (start 127.6 110.55) (end 127.6 117) (width 0.3) (layer "F.Cu") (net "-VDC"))
 (segment (start 130.1 128.3) (end 130.1 119.5) (width 0.3) (layer "F.Cu") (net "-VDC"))
 (segment (start 96.6 133.2) (end 97.75 134.35) (width 0.3) (layer "F.Cu") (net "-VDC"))
 (segment (start 104.79 100.81) (end 96.6 109) (width 0.3) (layer "F.Cu") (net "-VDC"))
 (segment (start 124.05 134.35) (end 130.1 128.3) (width 0.3) (layer "F.Cu") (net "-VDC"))
 (segment (start 106.94 100.81) (end 104.79 100.81) (width 0.3) (layer "F.Cu") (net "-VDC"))
 (segment (start 97.75 134.35) (end 124.05 134.35) (width 0.3) (layer "F.Cu") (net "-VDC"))
 (segment (start 96.6 109) (end 96.6 133.2) (width 0.3) (layer "F.Cu") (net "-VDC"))
 (segment (start 127.6 117) (end 130.1 119.5) (width 0.3) (layer "F.Cu") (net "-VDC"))
 (segment (start 111.97 85.46) (end 102 85.46) (width 0.3) (layer "F.Cu") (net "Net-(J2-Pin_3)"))
 (segment (start 114 87.49) (end 111.97 85.46) (width 0.3) (layer "F.Cu") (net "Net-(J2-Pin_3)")))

